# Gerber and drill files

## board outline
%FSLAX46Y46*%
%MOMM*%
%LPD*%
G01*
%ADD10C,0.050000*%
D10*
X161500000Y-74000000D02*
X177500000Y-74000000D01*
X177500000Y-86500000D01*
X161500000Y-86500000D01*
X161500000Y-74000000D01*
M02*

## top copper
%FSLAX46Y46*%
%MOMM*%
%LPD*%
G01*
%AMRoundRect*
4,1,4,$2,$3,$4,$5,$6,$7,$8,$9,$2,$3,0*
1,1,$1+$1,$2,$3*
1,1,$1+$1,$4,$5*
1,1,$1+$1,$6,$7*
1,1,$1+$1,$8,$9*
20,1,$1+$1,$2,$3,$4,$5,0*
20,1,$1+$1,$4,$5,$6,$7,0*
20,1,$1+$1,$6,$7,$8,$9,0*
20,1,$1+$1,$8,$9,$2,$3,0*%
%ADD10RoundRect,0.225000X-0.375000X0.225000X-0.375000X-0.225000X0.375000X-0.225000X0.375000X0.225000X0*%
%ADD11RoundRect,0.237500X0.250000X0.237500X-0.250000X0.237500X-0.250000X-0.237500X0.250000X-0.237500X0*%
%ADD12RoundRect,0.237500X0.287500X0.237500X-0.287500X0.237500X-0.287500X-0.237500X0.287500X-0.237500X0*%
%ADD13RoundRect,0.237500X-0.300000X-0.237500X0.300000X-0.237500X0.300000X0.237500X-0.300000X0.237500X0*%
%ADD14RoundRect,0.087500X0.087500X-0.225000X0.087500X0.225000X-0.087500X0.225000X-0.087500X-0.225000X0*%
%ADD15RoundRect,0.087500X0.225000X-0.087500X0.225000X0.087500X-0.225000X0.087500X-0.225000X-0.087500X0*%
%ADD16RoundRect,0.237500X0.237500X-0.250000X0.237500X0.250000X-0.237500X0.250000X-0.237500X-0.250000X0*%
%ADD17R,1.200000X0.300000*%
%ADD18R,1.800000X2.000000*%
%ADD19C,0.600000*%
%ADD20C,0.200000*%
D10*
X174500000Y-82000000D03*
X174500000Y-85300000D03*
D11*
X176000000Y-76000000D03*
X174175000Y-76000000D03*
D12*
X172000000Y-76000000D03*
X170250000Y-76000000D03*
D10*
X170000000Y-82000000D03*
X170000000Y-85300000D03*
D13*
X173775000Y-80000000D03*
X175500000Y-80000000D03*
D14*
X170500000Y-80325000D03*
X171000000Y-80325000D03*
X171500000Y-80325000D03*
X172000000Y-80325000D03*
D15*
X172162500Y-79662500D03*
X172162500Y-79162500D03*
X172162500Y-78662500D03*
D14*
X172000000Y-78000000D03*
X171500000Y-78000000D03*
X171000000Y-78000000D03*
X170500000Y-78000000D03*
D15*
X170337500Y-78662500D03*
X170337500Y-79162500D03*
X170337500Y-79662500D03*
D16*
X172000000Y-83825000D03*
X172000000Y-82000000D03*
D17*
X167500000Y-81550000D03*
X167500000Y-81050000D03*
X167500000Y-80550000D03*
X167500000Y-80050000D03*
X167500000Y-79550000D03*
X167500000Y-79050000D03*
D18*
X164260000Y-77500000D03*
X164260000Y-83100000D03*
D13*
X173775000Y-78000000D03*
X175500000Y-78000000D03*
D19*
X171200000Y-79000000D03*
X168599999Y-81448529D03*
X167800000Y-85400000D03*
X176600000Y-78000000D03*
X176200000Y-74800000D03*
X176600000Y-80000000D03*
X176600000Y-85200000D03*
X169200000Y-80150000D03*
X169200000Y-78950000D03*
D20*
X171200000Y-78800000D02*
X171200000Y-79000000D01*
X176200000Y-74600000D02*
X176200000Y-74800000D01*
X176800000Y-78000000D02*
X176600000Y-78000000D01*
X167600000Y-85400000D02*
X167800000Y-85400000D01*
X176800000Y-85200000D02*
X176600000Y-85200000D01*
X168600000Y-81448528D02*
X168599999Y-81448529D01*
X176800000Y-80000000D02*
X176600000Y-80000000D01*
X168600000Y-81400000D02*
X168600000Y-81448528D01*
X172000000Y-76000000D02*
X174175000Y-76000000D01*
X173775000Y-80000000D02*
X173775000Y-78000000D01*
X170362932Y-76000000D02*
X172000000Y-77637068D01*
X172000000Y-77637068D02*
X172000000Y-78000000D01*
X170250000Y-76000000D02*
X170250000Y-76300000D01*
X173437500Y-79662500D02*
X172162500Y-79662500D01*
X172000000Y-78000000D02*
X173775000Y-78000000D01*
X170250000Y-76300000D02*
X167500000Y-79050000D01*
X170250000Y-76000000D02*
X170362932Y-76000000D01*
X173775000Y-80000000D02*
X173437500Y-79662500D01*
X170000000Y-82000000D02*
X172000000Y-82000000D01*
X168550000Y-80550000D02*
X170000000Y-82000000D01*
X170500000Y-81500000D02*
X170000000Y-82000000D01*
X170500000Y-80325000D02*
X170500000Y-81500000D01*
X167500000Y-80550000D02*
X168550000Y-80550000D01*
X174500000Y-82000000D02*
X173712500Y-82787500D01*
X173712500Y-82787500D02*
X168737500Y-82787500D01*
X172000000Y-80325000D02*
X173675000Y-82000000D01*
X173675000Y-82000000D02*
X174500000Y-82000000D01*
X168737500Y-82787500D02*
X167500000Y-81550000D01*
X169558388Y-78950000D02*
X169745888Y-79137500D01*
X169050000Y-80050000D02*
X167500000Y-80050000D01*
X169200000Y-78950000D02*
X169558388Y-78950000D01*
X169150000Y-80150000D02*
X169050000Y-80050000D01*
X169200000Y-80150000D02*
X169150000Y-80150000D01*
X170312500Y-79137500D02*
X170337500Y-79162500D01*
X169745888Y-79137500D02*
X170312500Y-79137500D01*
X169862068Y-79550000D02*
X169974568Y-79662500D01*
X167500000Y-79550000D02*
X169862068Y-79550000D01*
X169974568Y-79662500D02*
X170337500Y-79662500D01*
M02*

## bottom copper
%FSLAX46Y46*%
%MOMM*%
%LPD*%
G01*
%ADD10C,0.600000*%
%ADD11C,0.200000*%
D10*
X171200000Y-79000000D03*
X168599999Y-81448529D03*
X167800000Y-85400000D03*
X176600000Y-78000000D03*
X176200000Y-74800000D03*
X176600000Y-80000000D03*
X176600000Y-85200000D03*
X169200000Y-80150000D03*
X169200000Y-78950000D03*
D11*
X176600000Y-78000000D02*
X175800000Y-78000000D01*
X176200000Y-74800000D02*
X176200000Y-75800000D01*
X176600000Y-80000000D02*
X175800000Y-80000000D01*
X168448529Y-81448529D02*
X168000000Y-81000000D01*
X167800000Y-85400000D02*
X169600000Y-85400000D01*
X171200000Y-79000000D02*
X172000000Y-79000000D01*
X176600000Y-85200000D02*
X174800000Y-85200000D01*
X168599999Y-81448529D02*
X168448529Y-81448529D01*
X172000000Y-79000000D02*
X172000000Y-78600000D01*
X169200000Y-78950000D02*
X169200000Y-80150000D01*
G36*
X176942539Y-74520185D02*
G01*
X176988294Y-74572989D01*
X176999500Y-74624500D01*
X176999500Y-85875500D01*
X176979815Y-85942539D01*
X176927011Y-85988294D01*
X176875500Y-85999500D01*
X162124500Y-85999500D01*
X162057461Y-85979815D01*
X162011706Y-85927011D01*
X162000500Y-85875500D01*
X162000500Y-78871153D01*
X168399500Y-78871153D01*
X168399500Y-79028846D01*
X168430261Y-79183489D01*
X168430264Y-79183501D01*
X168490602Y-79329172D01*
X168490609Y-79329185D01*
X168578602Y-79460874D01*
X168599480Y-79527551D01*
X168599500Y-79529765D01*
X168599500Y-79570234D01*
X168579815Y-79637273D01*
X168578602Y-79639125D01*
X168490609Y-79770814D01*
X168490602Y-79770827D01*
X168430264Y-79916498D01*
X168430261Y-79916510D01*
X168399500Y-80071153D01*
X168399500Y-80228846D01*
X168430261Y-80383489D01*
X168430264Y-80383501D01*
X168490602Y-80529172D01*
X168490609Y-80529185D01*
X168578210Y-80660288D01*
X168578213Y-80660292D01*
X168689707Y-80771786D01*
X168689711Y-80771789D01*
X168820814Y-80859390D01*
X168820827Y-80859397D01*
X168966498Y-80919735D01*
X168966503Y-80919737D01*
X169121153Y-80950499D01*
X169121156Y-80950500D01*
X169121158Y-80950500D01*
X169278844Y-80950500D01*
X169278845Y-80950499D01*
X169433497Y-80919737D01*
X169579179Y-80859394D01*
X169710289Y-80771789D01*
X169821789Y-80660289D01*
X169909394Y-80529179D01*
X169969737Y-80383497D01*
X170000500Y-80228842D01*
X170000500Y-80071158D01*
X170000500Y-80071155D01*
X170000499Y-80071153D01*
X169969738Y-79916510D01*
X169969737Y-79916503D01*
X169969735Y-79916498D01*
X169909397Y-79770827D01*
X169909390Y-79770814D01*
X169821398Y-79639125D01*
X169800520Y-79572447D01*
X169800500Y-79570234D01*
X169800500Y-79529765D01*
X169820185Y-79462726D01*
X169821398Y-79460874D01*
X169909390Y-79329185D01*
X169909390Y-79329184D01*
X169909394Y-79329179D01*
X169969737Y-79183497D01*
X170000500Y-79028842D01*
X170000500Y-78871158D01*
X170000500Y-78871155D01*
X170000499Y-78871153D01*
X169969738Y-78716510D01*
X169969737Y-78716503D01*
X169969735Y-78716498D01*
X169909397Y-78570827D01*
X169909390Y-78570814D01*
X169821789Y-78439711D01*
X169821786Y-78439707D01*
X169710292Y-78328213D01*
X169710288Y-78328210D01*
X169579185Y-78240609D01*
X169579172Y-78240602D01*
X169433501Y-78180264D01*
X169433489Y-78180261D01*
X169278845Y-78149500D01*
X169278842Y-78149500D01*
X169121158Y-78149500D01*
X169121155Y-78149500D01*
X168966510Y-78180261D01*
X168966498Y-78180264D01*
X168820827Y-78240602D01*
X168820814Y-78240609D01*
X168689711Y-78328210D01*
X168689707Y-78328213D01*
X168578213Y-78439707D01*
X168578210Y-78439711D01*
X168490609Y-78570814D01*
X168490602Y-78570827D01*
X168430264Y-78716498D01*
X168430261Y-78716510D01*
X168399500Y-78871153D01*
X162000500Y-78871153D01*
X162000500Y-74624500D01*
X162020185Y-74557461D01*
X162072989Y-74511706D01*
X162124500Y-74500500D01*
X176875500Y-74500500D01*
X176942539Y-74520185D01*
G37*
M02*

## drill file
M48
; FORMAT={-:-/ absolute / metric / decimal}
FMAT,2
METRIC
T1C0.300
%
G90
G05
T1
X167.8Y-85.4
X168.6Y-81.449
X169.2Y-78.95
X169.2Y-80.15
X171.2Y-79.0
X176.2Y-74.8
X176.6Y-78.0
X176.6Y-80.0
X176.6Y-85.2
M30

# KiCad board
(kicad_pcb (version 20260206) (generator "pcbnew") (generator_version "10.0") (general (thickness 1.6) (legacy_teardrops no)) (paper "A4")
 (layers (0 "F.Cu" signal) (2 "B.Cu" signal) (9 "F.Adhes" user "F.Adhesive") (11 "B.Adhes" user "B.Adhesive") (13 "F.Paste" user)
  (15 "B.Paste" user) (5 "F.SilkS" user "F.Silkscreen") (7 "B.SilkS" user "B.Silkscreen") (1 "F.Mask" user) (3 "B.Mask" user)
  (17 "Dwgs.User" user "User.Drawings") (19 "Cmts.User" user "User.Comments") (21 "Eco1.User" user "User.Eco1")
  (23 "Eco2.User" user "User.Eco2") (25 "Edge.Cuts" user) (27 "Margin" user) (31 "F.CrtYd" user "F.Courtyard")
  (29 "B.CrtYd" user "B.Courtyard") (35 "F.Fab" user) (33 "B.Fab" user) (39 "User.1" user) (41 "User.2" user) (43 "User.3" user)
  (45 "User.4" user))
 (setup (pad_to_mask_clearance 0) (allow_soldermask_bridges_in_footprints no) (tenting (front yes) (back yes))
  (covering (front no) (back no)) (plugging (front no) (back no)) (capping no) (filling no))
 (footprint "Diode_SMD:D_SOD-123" (layer "F.Cu") (at 174.5 83.65 -90)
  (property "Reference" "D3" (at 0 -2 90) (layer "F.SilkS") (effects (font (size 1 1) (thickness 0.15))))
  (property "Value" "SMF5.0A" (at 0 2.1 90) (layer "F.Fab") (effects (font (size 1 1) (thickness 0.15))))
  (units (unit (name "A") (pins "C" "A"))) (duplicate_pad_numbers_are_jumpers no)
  (pad "1" smd roundrect (at -1.65 0 270) (size 0.9 1.2) (layers "F.Cu" "F.Mask" "F.Paste") (roundrect_rratio 0.25) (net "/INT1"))
  (pad "2" smd roundrect (at 1.65 0 270) (size 0.9 1.2) (layers "F.Cu" "F.Mask" "F.Paste") (roundrect_rratio 0.25) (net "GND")))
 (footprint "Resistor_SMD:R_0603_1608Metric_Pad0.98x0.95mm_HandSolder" (layer "F.Cu") (at 175.0875 76 180)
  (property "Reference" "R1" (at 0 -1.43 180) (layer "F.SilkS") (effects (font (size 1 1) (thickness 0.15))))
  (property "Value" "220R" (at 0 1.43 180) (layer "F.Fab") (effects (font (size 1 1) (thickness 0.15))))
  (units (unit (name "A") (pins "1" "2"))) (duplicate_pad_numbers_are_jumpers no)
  (pad "1" smd roundrect (at -0.9125 0 180) (size 0.975 0.95) (layers "F.Cu" "F.Mask" "F.Paste") (roundrect_rratio 0.25) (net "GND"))
  (pad "2" smd roundrect (at 0.9125 0 180) (size 0.975 0.95) (layers "F.Cu" "F.Mask" "F.Paste") (roundrect_rratio 0.25) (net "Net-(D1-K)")))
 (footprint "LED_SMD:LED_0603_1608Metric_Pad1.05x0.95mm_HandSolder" (layer "F.Cu") (at 171.125 76 180)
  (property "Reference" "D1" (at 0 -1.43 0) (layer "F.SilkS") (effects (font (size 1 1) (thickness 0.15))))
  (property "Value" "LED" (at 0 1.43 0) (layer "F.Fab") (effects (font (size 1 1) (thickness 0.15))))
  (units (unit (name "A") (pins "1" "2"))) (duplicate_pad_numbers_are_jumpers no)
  (pad "1" smd roundrect (at -0.875 0 180) (size 1.05 0.95) (layers "F.Cu" "F.Mask" "F.Paste") (roundrect_rratio 0.25) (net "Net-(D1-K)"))
  (pad "2" smd roundrect (at 0.875 0 180) (size 1.05 0.95) (layers "F.Cu" "F.Mask" "F.Paste") (roundrect_rratio 0.25) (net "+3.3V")))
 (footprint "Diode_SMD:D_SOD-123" (layer "F.Cu") (at 170 83.65 -90)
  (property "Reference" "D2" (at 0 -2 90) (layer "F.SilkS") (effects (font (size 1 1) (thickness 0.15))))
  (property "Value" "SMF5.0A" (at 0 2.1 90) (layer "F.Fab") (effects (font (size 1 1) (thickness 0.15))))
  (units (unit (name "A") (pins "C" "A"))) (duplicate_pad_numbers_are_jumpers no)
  (pad "1" smd roundrect (at -1.65 0 270) (size 0.9 1.2) (layers "F.Cu" "F.Mask" "F.Paste") (roundrect_rratio 0.25) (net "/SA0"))
  (pad "2" smd roundrect (at 1.65 0 270) (size 0.9 1.2) (layers "F.Cu" "F.Mask" "F.Paste") (roundrect_rratio 0.25) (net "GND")))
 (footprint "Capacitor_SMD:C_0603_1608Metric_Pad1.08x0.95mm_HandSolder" (layer "F.Cu") (at 174.6375 80)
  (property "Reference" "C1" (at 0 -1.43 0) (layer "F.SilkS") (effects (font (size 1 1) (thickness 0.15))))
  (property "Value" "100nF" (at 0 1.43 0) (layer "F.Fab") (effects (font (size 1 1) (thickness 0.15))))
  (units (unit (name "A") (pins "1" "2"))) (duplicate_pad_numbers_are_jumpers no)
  (pad "1" smd roundrect (at -0.8625 0) (size 1.075 0.95) (layers "F.Cu" "F.Mask" "F.Paste") (roundrect_rratio 0.25) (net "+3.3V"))
  (pad "2" smd roundrect (at 0.8625 0) (size 1.075 0.95) (layers "F.Cu" "F.Mask" "F.Paste") (roundrect_rratio 0.25) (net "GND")))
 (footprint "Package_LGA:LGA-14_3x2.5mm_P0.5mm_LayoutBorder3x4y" (layer "F.Cu") (at 171.25 79.1625 90)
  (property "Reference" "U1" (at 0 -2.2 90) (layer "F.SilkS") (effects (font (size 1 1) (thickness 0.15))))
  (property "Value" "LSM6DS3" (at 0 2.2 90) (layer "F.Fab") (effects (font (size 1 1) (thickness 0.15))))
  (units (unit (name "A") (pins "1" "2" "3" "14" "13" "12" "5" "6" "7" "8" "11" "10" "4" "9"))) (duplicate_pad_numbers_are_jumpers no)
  (pad "1" smd roundrect (at -1.1625 -0.75 90) (size 0.625 0.35) (layers "F.Cu" "F.Mask" "F.Paste") (roundrect_rratio 0.25) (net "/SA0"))
  (pad "2" smd roundrect (at -1.1625 -0.25 90) (size 0.625 0.35) (layers "F.Cu" "F.Mask" "F.Paste") (roundrect_rratio 0.25)
   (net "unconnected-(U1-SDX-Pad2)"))
  (pad "3" smd roundrect (at -1.1625 0.25 90) (size 0.625 0.35) (layers "F.Cu" "F.Mask" "F.Paste") (roundrect_rratio 0.25)
   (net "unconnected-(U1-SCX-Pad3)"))
  (pad "4" smd roundrect (at -1.1625 0.75 90) (size 0.625 0.35) (layers "F.Cu" "F.Mask" "F.Paste") (roundrect_rratio 0.25) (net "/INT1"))
  (pad "5" smd roundrect (at -0.5 0.9125 90) (size 0.35 0.625) (layers "F.Cu" "F.Mask" "F.Paste") (roundrect_rratio 0.25) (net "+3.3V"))
  (pad "6" smd roundrect (at 0 0.9125 90) (size 0.35 0.625) (layers "F.Cu" "F.Mask" "F.Paste") (roundrect_rratio 0.25) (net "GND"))
  (pad "7" smd roundrect (at 0.5 0.9125 90) (size 0.35 0.625) (layers "F.Cu" "F.Mask" "F.Paste") (roundrect_rratio 0.25) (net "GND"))
  (pad "8" smd roundrect (at 1.1625 0.75 90) (size 0.625 0.35) (layers "F.Cu" "F.Mask" "F.Paste") (roundrect_rratio 0.25) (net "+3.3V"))
  (pad "9" smd roundrect (at 1.1625 0.25 90) (size 0.625 0.35) (layers "F.Cu" "F.Mask" "F.Paste") (roundrect_rratio 0.25)
   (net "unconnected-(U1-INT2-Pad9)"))
  (pad "10" smd roundrect (at 1.1625 -0.25 90) (size 0.625 0.35) (layers "F.Cu" "F.Mask" "F.Paste") (roundrect_rratio 0.25)
   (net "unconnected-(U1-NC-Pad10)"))
  (pad "11" smd roundrect (at 1.1625 -0.75 90) (size 0.625 0.35) (layers "F.Cu" "F.Mask" "F.Paste") (roundrect_rratio 0.25)
   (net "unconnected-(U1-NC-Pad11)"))
  (pad "12" smd roundrect (at 0.5 -0.9125 90) (size 0.35 0.625) (layers "F.Cu" "F.Mask" "F.Paste") (roundrect_rratio 0.25)
   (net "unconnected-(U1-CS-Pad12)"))
  (pad "13" smd roundrect (at 0 -0.9125 90) (size 0.35 0.625) (layers "F.Cu" "F.Mask" "F.Paste") (roundrect_rratio 0.25) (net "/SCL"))
  (pad "14" smd roundrect (at -0.5 -0.9125 90) (size 0.35 0.625) (layers "F.Cu" "F.Mask" "F.Paste") (roundrect_rratio 0.25) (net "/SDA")))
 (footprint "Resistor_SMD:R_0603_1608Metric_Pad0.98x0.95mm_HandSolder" (layer "F.Cu") (at 172 82.9125 90)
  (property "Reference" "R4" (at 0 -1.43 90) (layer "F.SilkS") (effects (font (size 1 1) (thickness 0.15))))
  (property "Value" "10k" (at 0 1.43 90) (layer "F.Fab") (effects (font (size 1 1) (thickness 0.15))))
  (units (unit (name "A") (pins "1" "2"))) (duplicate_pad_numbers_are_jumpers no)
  (pad "1" smd roundrect (at -0.9125 0 90) (size 0.975 0.95) (layers "F.Cu" "F.Mask" "F.Paste") (roundrect_rratio 0.25) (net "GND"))
  (pad "2" smd roundrect (at 0.9125 0 90) (size 0.975 0.95) (layers "F.Cu" "F.Mask" "F.Paste") (roundrect_rratio 0.25) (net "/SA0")))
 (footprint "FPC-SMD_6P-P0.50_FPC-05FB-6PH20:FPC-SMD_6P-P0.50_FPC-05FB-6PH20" (layer "F.Cu") (at 165.88 80.3 -90)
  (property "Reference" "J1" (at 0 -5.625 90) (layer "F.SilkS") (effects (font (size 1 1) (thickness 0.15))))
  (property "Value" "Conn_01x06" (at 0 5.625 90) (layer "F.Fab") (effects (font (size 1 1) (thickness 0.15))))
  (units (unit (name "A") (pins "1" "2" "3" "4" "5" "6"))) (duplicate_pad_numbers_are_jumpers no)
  (pad "1" smd rect (at 1.25 -1.62 270) (size 0.3 1.2) (layers "F.Cu" "F.Mask" "F.Paste") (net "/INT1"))
  (pad "2" smd rect (at 0.75 -1.62 270) (size 0.3 1.2) (layers "F.Cu" "F.Mask" "F.Paste") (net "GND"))
  (pad "3" smd rect (at 0.25 -1.62 270) (size 0.3 1.2) (layers "F.Cu" "F.Mask" "F.Paste") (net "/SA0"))
  (pad "4" smd rect (at -0.25 -1.62 270) (size 0.3 1.2) (layers "F.Cu" "F.Mask" "F.Paste") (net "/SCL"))
  (pad "5" smd rect (at -0.75 -1.62 270) (size 0.3 1.2) (layers "F.Cu" "F.Mask" "F.Paste") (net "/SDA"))
  (pad "6" smd rect (at -1.25 -1.62 270) (size 0.3 1.2) (layers "F.Cu" "F.Mask" "F.Paste") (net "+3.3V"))
  (pad "7" smd rect (at -2.8 1.62 270) (size 2 1.8) (layers "F.Cu" "F.Mask" "F.Paste"))
  (pad "8" smd rect (at 2.8 1.62 270) (size 2 1.8) (layers "F.Cu" "F.Mask" "F.Paste")))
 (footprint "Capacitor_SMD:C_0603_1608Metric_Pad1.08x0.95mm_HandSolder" (layer "F.Cu") (at 174.6375 78)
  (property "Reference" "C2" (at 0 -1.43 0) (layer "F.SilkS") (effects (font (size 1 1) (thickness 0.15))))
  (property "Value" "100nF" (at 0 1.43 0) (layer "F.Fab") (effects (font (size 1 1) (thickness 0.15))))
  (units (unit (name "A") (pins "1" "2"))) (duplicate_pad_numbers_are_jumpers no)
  (pad "1" smd roundrect (at -0.8625 0) (size 1.075 0.95) (layers "F.Cu" "F.Mask" "F.Paste") (roundrect_rratio 0.25) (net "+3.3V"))
  (pad "2" smd roundrect (at 0.8625 0) (size 1.075 0.95) (layers "F.Cu" "F.Mask" "F.Paste") (roundrect_rratio 0.25) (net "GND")))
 (gr_rect (start 161.5 74) (end 177.5 86.5) (stroke (width 0.05) (type default)) (fill no) (layer "Edge.Cuts"))
 (segment (start 171.2 78.8) (end 171.2 79) (width 0.2) (layer "F.Cu") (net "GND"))
 (segment (start 176.2 74.6) (end 176.2 74.8) (width 0.2) (layer "F.Cu") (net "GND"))
 (segment (start 176.8 78) (end 176.6 78) (width 0.2) (layer "F.Cu") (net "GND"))
 (segment (start 167.6 85.4) (end 167.8 85.4) (width 0.2) (layer "F.Cu") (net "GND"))
 (segment (start 176.8 85.2) (end 176.6 85.2) (width 0.2) (layer "F.Cu") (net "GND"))
 (segment (start 168.6 81.448528) (end 168.599999 81.448529) (width 0.2) (layer "F.Cu") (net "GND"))
 (segment (start 176.8 80) (end 176.6 80) (width 0.2) (layer "F.Cu") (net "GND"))
 (segment (start 168.6 81.4) (end 168.6 81.448528) (width 0.2) (layer "F.Cu") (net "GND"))
 (via (at 171.2 79) (size 0.6) (drill 0.3) (layers "F.Cu" "B.Cu") (free yes) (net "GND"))
 (via (at 168.599999 81.448529) (size 0.6) (drill 0.3) (layers "F.Cu" "B.Cu") (free yes) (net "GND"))
 (via (at 167.8 85.4) (size 0.6) (drill 0.3) (layers "F.Cu" "B.Cu") (free yes) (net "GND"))
 (via (at 176.6 78) (size 0.6) (drill 0.3) (layers "F.Cu" "B.Cu") (free yes) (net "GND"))
 (via (at 176.2 74.8) (size 0.6) (drill 0.3) (layers "F.Cu" "B.Cu") (free yes) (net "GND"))
 (via (at 176.6 80) (size 0.6) (drill 0.3) (layers "F.Cu" "B.Cu") (free yes) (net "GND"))
 (via (at 176.6 85.2) (size 0.6) (drill 0.3) (layers "F.Cu" "B.Cu") (free yes) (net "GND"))
 (segment (start 176.6 78) (end 175.8 78) (width 0.2) (layer "B.Cu") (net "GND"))
 (segment (start 176.2 74.8) (end 176.2 75.8) (width 0.2) (layer "B.Cu") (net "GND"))
 (segment (start 176.6 80) (end 175.8 80) (width 0.2) (layer "B.Cu") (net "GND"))
 (segment (start 168.448529 81.448529) (end 168 81) (width 0.2) (layer "B.Cu") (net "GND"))
 (segment (start 167.8 85.4) (end 169.6 85.4) (width 0.2) (layer "B.Cu") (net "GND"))
 (segment (start 171.2 79) (end 172 79) (width 0.2) (layer "B.Cu") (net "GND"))
 (segment (start 176.6 85.2) (end 174.8 85.2) (width 0.2) (layer "B.Cu") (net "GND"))
 (segment (start 168.599999 81.448529) (end 168.448529 81.448529) (width 0.2) (layer "B.Cu") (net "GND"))
 (segment (start 172 79) (end 172 78.6) (width 0.2) (layer "B.Cu") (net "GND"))
 (segment (start 172 76) (end 174.175 76) (width 0.2) (layer "F.Cu") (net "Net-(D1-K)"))
 (segment (start 173.775 80) (end 173.775 78) (width 0.2) (layer "F.Cu") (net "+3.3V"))
 (segment (start 170.362932 76) (end 172 77.637068) (width 0.2) (layer "F.Cu") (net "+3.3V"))
 (segment (start 172 77.637068) (end 172 78) (width 0.2) (layer "F.Cu") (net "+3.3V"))
 (segment (start 170.25 76) (end 170.25 76.3) (width 0.2) (layer "F.Cu") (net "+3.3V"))
 (segment (start 173.4375 79.6625) (end 172.1625 79.6625) (width 0.2) (layer "F.Cu") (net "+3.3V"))
 (segment (start 172 78) (end 173.775 78) (width 0.2) (layer "F.Cu") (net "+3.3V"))
 (segment (start 170.25 76.3) (end 167.5 79.05) (width 0.2) (layer "F.Cu") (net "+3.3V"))
 (segment (start 170.25 76) (end 170.362932 76) (width 0.2) (layer "F.Cu") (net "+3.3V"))
 (segment (start 173.775 80) (end 173.4375 79.6625) (width 0.2) (layer "F.Cu") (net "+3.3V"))
 (segment (start 170 82) (end 172 82) (width 0.2) (layer "F.Cu") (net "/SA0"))
 (segment (start 168.55 80.55) (end 170 82) (width 0.2) (layer "F.Cu") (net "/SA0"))
 (segment (start 170.5 81.5) (end 170 82) (width 0.2) (layer "F.Cu") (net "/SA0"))
 (segment (start 170.5 80.325) (end 170.5 81.5) (width 0.2) (layer "F.Cu") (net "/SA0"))
 (segment (start 167.5 80.55) (end 168.55 80.55) (width 0.2) (layer "F.Cu") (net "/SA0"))
 (segment (start 174.5 82) (end 173.7125 82.7875) (width 0.2) (layer "F.Cu") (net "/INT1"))
 (segment (start 173.7125 82.7875) (end 168.7375 82.7875) (width 0.2) (layer "F.Cu") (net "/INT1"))
 (segment (start 172 80.325) (end 173.675 82) (width 0.2) (layer "F.Cu") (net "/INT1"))
 (segment (start 173.675 82) (end 174.5 82) (width 0.2) (layer "F.Cu") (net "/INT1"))
 (segment (start 168.7375 82.7875) (end 167.5 81.55) (width 0.2) (layer "F.Cu") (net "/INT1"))
 (segment (start 169.558388 78.95) (end 169.745888 79.1375) (width 0.2) (layer "F.Cu") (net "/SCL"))
 (segment (start 169.05 80.05) (end 167.5 80.05) (width 0.2) (layer "F.Cu") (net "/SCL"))
 (segment (start 169.2 78.95) (end 169.558388 78.95) (width 0.2) (layer "F.Cu") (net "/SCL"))
 (segment (start 169.15 80.15) (end 169.05 80.05) (width 0.2) (layer "F.Cu") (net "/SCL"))
 (segment (start 169.2 80.15) (end 169.15 80.15) (width 0.2) (layer "F.Cu") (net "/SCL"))
 (segment (start 170.3125 79.1375) (end 170.3375 79.1625) (width 0.2) (layer "F.Cu") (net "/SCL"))
 (segment (start 169.745888 79.1375) (end 170.3125 79.1375) (width 0.2) (layer "F.Cu") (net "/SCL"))
 (via (at 169.2 80.15) (size 0.6) (drill 0.3) (layers "F.Cu" "B.Cu") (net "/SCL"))
 (via (at 169.2 78.95) (size 0.6) (drill 0.3) (layers "F.Cu" "B.Cu") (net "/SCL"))
 (segment (start 169.2 78.95) (end 169.2 80.15) (width 0.2) (layer "B.Cu") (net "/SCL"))
 (segment (start 169.862068 79.55) (end 169.974568 79.6625) (width 0.2) (layer "F.Cu") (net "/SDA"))
 (segment (start 167.5 79.55) (end 169.862068 79.55) (width 0.2) (layer "F.Cu") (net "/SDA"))
 (segment (start 169.974568 79.6625) (end 170.3375 79.6625) (width 0.2) (layer "F.Cu") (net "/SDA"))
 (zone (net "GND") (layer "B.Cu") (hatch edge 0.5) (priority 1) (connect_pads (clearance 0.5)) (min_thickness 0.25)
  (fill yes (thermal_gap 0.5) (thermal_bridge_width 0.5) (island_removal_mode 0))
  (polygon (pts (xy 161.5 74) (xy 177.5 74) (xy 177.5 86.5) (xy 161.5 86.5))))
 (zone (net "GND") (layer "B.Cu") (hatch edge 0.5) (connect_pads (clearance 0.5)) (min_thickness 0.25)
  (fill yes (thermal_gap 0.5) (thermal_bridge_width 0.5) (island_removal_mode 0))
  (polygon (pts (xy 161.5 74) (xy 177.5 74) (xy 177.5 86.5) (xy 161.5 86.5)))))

